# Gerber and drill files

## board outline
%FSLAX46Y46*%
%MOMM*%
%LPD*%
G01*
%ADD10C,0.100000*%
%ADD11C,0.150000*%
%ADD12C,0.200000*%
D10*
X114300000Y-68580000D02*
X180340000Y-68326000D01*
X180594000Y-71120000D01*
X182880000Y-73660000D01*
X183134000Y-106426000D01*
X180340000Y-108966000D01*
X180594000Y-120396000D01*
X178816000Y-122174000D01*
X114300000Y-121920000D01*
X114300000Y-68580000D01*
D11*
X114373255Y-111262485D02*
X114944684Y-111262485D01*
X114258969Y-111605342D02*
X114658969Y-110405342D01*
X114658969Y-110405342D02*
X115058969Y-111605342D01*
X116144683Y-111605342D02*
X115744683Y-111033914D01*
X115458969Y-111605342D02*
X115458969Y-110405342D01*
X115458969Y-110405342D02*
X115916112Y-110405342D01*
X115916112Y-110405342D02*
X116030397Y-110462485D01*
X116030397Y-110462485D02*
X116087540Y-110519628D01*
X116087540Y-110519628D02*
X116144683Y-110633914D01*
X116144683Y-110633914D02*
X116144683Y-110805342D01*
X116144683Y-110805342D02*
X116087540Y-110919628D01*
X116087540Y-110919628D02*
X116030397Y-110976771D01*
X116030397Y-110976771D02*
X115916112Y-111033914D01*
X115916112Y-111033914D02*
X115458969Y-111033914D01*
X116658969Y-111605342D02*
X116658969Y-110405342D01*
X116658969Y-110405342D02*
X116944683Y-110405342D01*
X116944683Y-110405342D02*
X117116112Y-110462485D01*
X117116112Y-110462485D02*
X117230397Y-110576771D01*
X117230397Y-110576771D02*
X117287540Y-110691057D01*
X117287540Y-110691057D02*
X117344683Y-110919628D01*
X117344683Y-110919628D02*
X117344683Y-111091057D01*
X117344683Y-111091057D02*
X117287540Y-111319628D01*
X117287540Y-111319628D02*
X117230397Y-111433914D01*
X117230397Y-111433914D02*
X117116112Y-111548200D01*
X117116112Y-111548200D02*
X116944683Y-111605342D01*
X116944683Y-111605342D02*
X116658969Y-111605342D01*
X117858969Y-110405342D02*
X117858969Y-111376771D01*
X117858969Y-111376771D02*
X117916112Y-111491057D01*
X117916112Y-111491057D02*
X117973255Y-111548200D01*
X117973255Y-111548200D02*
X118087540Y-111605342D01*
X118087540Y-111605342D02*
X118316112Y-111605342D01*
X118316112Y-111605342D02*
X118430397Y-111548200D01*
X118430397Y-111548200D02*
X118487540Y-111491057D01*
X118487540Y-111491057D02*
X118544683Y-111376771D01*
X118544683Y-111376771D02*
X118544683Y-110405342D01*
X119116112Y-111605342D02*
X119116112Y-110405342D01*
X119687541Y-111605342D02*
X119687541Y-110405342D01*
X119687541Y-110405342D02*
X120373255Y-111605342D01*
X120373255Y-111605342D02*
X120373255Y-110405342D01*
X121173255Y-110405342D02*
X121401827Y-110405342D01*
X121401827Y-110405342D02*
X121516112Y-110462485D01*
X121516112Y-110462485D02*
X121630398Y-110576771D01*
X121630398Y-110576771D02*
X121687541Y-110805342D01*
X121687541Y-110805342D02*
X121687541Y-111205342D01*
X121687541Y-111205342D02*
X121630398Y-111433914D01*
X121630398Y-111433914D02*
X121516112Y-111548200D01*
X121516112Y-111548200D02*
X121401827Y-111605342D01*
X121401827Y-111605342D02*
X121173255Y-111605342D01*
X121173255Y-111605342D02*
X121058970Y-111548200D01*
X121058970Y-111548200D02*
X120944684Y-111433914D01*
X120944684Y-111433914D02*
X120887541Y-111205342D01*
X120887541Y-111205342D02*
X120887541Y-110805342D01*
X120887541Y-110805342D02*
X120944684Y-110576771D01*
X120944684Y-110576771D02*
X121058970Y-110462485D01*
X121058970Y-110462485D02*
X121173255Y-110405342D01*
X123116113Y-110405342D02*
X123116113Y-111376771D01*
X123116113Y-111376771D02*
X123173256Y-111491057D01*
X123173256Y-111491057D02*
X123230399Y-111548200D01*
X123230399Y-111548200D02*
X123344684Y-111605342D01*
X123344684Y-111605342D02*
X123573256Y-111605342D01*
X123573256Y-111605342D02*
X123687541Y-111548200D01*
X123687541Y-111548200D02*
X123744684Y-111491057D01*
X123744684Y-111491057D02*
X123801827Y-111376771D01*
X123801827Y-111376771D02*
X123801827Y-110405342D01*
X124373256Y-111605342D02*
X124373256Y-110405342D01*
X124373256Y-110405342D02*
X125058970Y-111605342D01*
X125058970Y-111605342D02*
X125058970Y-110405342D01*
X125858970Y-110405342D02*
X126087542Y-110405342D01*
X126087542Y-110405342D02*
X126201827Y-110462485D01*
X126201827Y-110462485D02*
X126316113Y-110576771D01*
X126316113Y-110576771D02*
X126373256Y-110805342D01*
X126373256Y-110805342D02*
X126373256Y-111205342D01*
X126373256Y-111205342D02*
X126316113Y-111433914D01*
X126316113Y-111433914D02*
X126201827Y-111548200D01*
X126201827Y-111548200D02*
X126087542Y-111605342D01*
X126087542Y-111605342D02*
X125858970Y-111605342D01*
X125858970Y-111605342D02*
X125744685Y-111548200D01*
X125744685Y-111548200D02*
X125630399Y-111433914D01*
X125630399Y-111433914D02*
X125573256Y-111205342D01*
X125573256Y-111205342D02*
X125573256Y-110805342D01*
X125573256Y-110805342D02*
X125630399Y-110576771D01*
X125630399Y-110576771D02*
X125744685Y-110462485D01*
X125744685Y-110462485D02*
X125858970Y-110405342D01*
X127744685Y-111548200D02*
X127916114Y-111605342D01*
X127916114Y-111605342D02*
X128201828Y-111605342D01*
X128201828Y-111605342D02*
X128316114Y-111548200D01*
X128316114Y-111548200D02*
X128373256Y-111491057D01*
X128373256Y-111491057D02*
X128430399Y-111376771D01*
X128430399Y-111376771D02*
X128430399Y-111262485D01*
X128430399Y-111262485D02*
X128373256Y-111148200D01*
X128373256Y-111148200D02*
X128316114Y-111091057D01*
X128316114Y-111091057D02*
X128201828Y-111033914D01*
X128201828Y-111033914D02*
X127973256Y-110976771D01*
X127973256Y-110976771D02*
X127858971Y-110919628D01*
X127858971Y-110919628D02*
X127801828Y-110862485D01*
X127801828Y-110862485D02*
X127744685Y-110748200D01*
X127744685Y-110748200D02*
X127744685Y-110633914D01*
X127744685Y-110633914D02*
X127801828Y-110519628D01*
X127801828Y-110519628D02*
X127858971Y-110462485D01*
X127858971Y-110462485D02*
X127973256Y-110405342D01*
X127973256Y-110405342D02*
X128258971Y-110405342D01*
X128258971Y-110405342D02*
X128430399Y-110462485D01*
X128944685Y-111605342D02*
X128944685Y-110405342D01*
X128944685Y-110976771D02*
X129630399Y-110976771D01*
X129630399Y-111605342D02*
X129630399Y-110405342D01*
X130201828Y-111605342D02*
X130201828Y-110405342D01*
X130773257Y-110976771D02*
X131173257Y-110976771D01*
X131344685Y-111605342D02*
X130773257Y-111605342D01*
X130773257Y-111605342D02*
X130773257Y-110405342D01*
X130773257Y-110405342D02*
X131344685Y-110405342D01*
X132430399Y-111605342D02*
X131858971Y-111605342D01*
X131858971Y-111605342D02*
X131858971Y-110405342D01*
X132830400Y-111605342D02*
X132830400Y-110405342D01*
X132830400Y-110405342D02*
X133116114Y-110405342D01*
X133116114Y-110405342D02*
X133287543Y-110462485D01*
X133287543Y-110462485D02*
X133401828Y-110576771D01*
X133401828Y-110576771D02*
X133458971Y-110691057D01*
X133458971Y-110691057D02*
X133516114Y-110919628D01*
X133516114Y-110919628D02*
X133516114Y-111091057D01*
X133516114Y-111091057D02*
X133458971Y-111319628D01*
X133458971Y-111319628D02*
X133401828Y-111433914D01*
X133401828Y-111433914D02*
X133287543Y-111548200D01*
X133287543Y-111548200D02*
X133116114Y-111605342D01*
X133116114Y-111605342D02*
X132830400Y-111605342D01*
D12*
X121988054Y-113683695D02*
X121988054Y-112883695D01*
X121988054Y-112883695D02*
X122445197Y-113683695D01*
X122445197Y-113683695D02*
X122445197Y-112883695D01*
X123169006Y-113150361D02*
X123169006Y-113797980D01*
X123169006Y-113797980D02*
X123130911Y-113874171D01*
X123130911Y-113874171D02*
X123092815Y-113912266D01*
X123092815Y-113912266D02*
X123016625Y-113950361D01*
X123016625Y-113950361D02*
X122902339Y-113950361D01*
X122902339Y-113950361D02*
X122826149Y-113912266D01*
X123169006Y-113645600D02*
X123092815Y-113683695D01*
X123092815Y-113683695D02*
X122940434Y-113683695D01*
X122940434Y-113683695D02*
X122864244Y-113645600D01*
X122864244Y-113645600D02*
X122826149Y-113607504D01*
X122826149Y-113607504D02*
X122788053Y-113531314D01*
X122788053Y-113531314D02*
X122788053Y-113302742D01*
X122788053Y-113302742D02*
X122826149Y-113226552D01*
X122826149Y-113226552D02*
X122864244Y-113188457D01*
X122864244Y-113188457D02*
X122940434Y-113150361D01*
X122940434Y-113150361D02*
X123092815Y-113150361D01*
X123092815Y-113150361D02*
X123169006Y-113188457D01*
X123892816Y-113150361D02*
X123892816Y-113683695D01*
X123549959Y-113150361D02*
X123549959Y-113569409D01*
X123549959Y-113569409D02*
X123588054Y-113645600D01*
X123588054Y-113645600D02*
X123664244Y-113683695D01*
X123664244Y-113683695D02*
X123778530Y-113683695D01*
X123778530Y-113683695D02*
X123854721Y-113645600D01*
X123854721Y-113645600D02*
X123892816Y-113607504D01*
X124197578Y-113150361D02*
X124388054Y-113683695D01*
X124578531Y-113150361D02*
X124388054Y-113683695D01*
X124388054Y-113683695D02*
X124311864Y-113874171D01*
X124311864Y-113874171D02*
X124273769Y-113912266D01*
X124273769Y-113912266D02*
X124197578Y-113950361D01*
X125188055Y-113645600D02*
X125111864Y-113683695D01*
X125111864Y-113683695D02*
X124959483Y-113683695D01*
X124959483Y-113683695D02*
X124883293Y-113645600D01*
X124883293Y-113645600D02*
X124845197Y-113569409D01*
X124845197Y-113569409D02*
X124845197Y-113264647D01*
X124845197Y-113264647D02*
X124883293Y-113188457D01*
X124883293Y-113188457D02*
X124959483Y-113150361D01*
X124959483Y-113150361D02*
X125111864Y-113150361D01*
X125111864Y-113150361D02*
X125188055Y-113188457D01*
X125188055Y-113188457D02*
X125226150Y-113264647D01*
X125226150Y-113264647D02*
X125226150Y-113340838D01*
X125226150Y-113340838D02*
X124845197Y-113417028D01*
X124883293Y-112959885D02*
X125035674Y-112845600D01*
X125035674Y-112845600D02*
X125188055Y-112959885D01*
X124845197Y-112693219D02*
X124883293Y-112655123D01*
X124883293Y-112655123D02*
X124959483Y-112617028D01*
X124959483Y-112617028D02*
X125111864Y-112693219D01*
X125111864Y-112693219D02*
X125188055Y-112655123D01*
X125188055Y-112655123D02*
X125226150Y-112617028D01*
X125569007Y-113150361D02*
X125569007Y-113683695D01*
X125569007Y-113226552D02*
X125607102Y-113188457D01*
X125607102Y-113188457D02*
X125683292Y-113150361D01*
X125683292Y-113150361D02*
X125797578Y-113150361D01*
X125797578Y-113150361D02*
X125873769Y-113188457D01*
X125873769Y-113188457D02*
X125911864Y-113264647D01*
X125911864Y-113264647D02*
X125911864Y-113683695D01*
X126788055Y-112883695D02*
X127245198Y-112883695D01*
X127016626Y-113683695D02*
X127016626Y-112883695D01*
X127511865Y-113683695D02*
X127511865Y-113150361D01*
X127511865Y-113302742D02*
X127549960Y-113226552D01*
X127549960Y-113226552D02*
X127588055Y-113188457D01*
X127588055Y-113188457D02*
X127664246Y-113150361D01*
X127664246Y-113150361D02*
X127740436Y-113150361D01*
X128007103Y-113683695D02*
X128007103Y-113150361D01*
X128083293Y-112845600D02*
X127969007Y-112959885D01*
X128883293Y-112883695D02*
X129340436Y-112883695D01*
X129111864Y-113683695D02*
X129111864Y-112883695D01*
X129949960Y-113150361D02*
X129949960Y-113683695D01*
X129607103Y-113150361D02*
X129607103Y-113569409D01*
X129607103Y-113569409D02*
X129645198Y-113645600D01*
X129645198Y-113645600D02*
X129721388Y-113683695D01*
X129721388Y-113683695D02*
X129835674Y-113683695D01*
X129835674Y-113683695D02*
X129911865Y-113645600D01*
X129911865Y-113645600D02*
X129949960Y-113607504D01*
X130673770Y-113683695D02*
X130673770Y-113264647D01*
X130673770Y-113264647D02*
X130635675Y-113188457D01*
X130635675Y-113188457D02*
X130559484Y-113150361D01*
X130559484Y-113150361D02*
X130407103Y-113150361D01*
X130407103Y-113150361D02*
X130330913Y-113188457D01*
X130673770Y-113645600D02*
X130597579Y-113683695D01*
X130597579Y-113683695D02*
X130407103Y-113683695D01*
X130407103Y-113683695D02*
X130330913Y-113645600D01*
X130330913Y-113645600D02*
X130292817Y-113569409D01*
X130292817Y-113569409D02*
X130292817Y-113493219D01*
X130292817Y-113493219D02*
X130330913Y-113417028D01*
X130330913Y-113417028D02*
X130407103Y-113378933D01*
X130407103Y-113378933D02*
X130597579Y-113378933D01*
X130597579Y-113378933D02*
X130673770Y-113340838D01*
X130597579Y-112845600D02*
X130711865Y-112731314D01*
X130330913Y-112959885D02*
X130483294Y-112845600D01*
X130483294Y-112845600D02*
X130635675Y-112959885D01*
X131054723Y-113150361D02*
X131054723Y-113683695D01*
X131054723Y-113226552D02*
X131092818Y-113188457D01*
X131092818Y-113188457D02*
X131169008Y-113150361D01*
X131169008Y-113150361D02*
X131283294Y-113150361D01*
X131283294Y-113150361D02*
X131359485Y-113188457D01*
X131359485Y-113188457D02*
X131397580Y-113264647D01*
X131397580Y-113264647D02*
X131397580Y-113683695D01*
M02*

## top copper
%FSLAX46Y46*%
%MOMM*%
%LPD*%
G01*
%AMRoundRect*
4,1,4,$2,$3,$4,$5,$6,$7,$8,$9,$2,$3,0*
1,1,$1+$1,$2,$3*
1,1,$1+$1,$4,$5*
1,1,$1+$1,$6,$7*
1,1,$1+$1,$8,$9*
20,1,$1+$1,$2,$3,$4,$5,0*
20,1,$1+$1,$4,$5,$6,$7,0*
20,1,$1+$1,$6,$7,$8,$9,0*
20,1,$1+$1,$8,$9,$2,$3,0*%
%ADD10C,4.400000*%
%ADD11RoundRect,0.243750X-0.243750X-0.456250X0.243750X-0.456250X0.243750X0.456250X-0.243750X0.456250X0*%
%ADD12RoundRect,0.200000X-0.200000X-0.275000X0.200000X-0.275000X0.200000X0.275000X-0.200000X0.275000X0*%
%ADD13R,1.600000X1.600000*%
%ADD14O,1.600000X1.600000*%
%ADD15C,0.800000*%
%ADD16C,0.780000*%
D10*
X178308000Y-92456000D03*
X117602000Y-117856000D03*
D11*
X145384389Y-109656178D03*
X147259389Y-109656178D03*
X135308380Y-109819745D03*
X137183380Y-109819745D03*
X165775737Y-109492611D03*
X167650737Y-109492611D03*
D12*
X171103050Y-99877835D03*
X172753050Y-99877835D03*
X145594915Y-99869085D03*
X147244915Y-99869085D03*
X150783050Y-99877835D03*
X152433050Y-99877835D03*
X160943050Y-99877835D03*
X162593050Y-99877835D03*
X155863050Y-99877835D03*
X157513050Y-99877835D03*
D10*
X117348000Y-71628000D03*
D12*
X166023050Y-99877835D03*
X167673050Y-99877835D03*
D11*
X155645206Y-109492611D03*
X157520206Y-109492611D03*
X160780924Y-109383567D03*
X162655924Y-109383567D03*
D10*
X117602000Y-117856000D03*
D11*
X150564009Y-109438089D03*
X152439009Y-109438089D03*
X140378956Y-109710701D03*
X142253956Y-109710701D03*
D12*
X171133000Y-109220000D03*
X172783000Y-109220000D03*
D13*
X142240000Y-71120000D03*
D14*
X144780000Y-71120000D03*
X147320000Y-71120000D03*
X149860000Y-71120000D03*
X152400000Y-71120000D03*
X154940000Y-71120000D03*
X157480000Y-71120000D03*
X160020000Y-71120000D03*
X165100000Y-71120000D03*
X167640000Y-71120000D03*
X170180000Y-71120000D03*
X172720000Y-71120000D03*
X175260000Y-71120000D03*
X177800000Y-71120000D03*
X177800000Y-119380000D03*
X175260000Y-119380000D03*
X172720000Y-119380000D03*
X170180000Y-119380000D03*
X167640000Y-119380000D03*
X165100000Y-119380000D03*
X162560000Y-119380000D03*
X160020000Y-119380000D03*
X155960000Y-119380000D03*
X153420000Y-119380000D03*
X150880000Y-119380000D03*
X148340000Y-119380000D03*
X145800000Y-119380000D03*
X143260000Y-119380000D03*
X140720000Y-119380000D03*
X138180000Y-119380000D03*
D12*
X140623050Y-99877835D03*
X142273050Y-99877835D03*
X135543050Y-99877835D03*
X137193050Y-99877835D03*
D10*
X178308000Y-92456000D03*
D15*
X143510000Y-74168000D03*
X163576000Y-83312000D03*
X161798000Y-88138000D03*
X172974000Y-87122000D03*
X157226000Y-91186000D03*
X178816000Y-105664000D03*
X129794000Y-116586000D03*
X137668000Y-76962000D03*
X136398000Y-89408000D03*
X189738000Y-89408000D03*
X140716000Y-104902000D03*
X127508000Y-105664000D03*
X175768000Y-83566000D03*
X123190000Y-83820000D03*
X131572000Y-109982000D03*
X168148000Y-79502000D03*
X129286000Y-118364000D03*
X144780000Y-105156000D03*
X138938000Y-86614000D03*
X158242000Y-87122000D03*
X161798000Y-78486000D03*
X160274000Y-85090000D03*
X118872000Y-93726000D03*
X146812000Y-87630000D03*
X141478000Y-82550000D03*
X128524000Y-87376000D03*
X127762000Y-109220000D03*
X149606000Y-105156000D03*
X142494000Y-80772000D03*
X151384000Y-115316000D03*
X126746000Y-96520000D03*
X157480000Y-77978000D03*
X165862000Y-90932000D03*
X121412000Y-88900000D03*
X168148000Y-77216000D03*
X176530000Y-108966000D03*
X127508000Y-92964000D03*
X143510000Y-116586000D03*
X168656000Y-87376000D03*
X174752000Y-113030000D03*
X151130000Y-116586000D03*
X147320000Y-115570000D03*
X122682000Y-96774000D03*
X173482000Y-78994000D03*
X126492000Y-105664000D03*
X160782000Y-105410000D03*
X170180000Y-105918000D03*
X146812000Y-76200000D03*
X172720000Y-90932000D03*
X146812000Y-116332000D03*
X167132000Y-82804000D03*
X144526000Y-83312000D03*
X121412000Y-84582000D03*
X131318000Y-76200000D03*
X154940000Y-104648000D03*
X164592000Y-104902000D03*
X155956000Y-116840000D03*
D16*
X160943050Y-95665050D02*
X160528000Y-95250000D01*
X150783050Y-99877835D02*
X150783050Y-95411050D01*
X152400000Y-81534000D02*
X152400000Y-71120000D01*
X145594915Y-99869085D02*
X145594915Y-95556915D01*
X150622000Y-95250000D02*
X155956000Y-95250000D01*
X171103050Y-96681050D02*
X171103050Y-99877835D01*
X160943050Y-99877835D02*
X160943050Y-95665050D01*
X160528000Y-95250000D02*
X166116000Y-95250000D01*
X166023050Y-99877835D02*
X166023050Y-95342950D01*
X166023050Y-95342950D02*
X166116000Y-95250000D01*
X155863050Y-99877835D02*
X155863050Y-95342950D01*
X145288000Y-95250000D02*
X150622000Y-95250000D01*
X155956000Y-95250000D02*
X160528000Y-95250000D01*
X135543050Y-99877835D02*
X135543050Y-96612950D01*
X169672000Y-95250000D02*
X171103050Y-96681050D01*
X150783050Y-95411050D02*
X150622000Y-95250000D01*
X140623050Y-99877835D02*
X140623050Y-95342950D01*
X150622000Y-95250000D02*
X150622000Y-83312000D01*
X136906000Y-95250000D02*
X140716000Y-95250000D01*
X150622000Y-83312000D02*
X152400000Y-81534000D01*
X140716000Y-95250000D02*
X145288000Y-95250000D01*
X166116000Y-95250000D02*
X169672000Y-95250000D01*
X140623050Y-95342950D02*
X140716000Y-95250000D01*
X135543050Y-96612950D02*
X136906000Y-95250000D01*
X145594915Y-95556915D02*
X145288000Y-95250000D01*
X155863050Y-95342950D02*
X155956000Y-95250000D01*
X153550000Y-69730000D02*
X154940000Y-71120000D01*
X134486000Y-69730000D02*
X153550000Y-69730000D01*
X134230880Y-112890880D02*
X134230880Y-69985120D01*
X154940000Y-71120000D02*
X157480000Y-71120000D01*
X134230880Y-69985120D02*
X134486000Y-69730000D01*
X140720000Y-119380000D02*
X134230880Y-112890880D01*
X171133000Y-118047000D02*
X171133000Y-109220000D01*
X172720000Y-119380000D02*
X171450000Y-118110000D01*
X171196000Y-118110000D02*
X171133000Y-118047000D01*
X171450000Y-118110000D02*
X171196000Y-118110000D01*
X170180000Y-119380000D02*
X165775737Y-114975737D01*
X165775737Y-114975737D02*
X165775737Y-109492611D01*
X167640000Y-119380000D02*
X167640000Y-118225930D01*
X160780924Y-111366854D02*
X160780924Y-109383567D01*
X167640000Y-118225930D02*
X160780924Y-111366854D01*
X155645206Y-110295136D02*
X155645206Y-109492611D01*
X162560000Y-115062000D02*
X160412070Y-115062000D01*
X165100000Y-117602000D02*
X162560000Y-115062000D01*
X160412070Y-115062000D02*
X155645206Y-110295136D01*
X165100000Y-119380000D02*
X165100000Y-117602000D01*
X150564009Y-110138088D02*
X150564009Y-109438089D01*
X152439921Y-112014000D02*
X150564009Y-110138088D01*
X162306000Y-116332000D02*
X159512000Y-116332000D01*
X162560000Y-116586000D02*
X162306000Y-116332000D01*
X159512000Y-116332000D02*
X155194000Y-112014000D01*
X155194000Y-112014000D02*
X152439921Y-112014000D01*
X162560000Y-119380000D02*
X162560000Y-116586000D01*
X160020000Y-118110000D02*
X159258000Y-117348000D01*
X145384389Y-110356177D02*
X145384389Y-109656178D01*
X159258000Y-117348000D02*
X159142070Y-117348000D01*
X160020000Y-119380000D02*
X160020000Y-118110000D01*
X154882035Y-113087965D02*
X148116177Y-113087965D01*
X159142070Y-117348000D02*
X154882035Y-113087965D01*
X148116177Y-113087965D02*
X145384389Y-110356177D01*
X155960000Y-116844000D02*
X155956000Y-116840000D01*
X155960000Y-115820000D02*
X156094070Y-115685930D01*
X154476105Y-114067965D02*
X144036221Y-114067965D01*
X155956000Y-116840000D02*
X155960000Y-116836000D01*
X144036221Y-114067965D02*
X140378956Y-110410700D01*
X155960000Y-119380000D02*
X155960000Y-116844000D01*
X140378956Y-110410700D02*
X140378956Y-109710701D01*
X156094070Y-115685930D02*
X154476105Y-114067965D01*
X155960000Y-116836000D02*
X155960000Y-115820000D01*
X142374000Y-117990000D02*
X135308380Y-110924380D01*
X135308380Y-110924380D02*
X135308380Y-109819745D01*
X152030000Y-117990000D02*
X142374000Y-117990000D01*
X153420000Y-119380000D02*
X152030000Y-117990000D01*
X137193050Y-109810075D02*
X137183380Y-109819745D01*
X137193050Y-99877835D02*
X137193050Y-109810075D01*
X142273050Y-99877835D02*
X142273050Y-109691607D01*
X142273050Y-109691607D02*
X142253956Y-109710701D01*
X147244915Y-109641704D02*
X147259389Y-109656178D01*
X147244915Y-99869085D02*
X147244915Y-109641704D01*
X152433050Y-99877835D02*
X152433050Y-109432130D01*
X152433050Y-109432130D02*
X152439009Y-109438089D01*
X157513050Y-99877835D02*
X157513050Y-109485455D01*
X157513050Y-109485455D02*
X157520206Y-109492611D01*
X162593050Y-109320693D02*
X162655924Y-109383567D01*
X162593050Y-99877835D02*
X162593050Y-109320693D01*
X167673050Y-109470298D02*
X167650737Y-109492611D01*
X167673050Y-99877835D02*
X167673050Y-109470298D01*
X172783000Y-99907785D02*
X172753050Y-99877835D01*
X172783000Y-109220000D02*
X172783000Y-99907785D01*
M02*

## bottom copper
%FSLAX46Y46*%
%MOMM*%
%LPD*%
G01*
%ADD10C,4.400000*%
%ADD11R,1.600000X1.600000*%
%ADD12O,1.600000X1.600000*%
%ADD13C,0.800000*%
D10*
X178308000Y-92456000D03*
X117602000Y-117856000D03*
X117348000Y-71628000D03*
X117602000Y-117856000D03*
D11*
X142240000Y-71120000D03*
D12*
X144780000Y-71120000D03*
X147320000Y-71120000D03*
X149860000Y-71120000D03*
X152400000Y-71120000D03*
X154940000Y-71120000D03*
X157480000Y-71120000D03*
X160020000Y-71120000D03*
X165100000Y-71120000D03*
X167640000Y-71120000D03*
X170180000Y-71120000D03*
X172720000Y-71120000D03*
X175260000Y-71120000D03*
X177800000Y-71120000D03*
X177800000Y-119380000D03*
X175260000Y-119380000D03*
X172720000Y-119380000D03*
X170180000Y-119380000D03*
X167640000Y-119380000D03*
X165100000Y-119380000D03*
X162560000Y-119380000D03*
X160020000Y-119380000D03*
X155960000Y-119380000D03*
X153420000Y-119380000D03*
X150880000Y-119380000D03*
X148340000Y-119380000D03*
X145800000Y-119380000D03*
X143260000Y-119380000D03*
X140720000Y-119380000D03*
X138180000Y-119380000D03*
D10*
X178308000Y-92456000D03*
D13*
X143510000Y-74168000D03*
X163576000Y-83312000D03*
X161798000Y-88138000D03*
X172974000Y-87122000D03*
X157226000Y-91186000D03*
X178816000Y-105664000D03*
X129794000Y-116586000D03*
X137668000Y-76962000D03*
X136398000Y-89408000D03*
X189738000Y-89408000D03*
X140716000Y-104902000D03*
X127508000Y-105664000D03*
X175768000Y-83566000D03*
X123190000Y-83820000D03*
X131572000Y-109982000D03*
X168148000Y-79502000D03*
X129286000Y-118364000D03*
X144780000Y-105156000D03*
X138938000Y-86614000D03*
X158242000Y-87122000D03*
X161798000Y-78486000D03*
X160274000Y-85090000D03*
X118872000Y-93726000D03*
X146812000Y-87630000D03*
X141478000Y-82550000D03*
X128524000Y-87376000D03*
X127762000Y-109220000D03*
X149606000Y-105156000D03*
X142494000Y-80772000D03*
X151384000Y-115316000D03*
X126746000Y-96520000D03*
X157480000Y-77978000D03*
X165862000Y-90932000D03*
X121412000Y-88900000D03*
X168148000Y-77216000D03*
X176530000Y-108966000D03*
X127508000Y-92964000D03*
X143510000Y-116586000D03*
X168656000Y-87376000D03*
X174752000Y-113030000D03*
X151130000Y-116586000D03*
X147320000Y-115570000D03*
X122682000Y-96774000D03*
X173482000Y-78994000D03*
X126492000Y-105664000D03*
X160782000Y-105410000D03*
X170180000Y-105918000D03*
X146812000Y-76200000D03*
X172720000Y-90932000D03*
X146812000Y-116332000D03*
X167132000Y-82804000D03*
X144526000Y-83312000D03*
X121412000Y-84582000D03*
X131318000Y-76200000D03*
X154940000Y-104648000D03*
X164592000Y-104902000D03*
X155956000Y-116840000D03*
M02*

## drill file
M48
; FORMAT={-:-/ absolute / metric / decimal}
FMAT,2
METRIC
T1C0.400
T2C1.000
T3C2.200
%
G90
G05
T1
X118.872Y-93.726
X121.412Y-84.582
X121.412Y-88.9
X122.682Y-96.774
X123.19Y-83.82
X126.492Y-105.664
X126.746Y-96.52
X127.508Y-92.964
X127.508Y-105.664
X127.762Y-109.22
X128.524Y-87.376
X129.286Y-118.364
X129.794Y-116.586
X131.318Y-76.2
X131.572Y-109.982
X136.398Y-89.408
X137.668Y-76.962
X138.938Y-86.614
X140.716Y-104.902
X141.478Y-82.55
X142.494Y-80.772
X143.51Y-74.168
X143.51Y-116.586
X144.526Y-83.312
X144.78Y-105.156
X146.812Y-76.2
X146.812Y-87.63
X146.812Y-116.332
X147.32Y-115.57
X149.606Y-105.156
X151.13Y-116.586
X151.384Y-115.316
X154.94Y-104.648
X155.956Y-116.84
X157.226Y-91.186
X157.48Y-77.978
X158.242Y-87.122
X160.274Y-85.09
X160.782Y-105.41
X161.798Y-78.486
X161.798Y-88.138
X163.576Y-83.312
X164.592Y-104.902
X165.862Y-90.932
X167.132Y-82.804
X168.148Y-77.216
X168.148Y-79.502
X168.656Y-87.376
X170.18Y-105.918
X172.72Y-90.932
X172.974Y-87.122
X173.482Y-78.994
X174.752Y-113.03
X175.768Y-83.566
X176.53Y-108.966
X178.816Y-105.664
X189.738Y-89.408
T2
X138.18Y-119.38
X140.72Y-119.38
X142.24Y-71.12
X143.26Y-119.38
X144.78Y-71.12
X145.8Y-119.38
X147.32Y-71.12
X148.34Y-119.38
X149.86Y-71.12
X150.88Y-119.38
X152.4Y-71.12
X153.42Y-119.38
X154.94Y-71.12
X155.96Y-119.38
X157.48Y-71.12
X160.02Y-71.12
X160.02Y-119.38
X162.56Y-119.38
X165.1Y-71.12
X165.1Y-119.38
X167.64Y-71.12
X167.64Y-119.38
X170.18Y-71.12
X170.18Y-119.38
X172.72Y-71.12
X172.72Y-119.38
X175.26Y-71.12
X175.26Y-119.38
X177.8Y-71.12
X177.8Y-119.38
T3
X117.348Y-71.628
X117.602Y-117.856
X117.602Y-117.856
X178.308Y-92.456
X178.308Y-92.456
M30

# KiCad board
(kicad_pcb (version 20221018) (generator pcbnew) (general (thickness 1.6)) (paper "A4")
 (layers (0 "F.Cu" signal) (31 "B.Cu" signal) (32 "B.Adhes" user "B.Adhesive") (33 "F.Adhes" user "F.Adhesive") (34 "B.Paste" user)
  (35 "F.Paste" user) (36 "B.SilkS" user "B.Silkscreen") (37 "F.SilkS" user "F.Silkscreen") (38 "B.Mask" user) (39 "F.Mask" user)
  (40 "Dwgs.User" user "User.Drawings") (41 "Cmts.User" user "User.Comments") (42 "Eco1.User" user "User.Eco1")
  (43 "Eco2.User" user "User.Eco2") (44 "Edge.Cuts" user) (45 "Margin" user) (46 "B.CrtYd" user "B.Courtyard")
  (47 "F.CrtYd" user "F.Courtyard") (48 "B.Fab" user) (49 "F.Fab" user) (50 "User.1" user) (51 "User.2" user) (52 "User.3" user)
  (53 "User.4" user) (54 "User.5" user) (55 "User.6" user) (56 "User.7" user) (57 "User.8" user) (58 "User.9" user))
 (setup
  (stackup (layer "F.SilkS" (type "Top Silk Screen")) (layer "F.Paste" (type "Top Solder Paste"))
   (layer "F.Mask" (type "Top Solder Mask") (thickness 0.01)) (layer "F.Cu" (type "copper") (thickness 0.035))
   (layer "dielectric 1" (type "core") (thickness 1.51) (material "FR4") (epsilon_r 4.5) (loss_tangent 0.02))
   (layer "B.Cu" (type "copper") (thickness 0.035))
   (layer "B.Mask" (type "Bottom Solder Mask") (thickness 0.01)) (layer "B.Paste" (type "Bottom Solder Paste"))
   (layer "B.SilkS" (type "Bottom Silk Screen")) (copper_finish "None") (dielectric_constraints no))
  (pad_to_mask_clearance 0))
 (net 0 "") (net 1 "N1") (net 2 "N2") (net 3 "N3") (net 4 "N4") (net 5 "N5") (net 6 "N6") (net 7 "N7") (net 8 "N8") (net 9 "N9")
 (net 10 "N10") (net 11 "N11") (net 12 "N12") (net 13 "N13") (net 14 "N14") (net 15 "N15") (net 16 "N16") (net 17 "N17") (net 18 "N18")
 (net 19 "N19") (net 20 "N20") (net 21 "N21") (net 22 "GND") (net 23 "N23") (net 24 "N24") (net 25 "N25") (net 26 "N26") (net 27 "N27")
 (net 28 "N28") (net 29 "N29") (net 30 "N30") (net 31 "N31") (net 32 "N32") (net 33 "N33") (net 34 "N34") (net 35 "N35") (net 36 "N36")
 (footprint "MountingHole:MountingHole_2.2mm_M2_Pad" (layer "F.Cu") (at 178.308 92.456)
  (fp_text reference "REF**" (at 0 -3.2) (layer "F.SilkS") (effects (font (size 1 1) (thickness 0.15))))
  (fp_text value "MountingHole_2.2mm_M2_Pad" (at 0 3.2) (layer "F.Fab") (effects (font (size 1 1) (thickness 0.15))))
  (pad "1" thru_hole circle (at 0 0) (size 4.4 4.4) (drill 2.2) (layers "*.Cu" "*.Mask")))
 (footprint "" (layer "F.Cu") (at 117.602 117.856)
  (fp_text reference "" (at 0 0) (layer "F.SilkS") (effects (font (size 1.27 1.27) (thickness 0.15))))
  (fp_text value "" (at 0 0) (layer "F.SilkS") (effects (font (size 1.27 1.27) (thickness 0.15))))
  (pad "1" thru_hole circle (at 0 0) (size 4.4 4.4) (drill 2.2) (layers "*.Cu" "*.Mask")))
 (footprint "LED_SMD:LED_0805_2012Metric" (layer "F.Cu") (at 146.321889 109.656178)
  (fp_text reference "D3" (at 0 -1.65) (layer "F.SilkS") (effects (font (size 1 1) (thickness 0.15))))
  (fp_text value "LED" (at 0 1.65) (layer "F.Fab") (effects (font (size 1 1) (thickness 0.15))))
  (pad "1" smd roundrect (at -0.9375 0) (size 0.975 1.4) (layers "F.Cu" "F.Paste" "F.Mask") (roundrect_rratio 0.25) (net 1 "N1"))
  (pad "2" smd roundrect (at 0.9375 0) (size 0.975 1.4) (layers "F.Cu" "F.Paste" "F.Mask") (roundrect_rratio 0.25) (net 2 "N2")))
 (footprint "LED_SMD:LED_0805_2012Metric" (layer "F.Cu") (at 136.24588 109.819745)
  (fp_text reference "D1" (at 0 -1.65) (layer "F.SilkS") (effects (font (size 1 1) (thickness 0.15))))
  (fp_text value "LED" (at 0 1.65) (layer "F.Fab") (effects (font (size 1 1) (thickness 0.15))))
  (pad "1" smd roundrect (at -0.9375 0) (size 0.975 1.4) (layers "F.Cu" "F.Paste" "F.Mask") (roundrect_rratio 0.25) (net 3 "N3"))
  (pad "2" smd roundrect (at 0.9375 0) (size 0.975 1.4) (layers "F.Cu" "F.Paste" "F.Mask") (roundrect_rratio 0.25) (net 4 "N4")))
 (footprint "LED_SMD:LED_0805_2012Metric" (layer "F.Cu") (at 166.713237 109.492611)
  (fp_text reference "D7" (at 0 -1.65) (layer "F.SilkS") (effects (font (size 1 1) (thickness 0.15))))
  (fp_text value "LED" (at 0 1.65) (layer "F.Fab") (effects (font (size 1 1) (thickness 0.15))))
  (pad "1" smd roundrect (at -0.9375 0) (size 0.975 1.4) (layers "F.Cu" "F.Paste" "F.Mask") (roundrect_rratio 0.25) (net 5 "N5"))
  (pad "2" smd roundrect (at 0.9375 0) (size 0.975 1.4) (layers "F.Cu" "F.Paste" "F.Mask") (roundrect_rratio 0.25) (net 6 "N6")))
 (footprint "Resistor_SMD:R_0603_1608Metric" (layer "F.Cu") (at 171.92805 99.877835)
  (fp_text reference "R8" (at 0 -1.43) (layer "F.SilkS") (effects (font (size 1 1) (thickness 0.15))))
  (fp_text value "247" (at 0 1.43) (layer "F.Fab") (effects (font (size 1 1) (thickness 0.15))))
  (pad "1" smd roundrect (at -0.825 0) (size 0.8 0.95) (layers "F.Cu" "F.Paste" "F.Mask") (roundrect_rratio 0.25) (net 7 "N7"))
  (pad "2" smd roundrect (at 0.825 0) (size 0.8 0.95) (layers "F.Cu" "F.Paste" "F.Mask") (roundrect_rratio 0.25) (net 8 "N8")))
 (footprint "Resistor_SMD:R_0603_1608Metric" (layer "F.Cu") (at 146.419915 99.869085)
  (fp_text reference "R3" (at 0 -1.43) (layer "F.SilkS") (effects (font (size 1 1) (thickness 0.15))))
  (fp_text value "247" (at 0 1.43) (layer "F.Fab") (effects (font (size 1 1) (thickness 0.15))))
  (pad "1" smd roundrect (at -0.825 0) (size 0.8 0.95) (layers "F.Cu" "F.Paste" "F.Mask") (roundrect_rratio 0.25) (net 7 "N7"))
  (pad "2" smd roundrect (at 0.825 0) (size 0.8 0.95) (layers "F.Cu" "F.Paste" "F.Mask") (roundrect_rratio 0.25) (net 2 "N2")))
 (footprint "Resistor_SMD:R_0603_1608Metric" (layer "F.Cu") (at 151.60805 99.877835)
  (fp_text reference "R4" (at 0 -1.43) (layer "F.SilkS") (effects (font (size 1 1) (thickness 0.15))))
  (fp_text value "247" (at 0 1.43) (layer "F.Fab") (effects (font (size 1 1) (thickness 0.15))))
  (pad "1" smd roundrect (at -0.825 0) (size 0.8 0.95) (layers "F.Cu" "F.Paste" "F.Mask") (roundrect_rratio 0.25) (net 7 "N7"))
  (pad "2" smd roundrect (at 0.825 0) (size 0.8 0.95) (layers "F.Cu" "F.Paste" "F.Mask") (roundrect_rratio 0.25) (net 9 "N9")))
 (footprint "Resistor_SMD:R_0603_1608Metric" (layer "F.Cu") (at 161.76805 99.877835)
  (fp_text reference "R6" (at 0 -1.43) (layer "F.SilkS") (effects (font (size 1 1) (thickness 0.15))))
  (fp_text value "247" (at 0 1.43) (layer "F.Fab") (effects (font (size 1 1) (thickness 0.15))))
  (pad "1" smd roundrect (at -0.825 0) (size 0.8 0.95) (layers "F.Cu" "F.Paste" "F.Mask") (roundrect_rratio 0.25) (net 7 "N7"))
  (pad "2" smd roundrect (at 0.825 0) (size 0.8 0.95) (layers "F.Cu" "F.Paste" "F.Mask") (roundrect_rratio 0.25) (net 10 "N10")))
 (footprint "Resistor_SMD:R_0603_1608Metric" (layer "F.Cu") (at 156.68805 99.877835)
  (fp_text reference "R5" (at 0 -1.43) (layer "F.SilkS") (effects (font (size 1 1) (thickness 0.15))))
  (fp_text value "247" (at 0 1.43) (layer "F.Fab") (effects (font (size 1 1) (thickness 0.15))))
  (pad "1" smd roundrect (at -0.825 0) (size 0.8 0.95) (layers "F.Cu" "F.Paste" "F.Mask") (roundrect_rratio 0.25) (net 7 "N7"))
  (pad "2" smd roundrect (at 0.825 0) (size 0.8 0.95) (layers "F.Cu" "F.Paste" "F.Mask") (roundrect_rratio 0.25) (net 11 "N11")))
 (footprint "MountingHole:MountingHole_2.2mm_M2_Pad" (layer "F.Cu") (at 117.348 71.628)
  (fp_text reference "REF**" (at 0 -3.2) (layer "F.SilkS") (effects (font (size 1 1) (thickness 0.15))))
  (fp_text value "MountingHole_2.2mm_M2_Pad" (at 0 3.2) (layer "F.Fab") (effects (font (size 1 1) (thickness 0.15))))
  (pad "1" thru_hole circle (at 0 0) (size 4.4 4.4) (drill 2.2) (layers "*.Cu" "*.Mask")))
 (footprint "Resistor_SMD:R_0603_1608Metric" (layer "F.Cu") (at 166.84805 99.877835)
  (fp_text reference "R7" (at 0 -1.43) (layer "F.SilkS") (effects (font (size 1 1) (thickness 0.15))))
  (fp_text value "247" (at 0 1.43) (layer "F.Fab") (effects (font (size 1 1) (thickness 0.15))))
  (pad "1" smd roundrect (at -0.825 0) (size 0.8 0.95) (layers "F.Cu" "F.Paste" "F.Mask") (roundrect_rratio 0.25) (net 7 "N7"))
  (pad "2" smd roundrect (at 0.825 0) (size 0.8 0.95) (layers "F.Cu" "F.Paste" "F.Mask") (roundrect_rratio 0.25) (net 6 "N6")))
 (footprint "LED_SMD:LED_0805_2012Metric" (layer "F.Cu") (at 156.582706 109.492611)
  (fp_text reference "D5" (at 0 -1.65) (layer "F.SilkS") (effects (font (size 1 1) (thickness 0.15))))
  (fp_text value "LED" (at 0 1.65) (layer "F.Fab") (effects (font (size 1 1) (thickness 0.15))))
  (pad "1" smd roundrect (at -0.9375 0) (size 0.975 1.4) (layers "F.Cu" "F.Paste" "F.Mask") (roundrect_rratio 0.25) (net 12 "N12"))
  (pad "2" smd roundrect (at 0.9375 0) (size 0.975 1.4) (layers "F.Cu" "F.Paste" "F.Mask") (roundrect_rratio 0.25) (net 11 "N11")))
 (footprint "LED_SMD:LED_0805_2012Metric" (layer "F.Cu") (at 161.718424 109.383567)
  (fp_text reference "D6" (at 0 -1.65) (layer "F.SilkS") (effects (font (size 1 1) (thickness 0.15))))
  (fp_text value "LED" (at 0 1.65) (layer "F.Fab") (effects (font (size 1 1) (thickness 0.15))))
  (pad "1" smd roundrect (at -0.9375 0) (size 0.975 1.4) (layers "F.Cu" "F.Paste" "F.Mask") (roundrect_rratio 0.25) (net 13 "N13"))
  (pad "2" smd roundrect (at 0.9375 0) (size 0.975 1.4) (layers "F.Cu" "F.Paste" "F.Mask") (roundrect_rratio 0.25) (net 10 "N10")))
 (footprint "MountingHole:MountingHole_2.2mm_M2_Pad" (layer "F.Cu") (at 117.602 117.856)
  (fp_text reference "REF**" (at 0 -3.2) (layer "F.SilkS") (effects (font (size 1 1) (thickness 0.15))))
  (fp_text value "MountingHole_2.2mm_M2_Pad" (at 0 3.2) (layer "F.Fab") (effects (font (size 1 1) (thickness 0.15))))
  (pad "1" thru_hole circle (at 0 0) (size 4.4 4.4) (drill 2.2) (layers "*.Cu" "*.Mask")))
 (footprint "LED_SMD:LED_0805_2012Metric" (layer "F.Cu") (at 151.501509 109.438089)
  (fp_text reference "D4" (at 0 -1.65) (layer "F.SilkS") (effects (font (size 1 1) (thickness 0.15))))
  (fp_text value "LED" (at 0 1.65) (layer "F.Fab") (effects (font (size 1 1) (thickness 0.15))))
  (pad "1" smd roundrect (at -0.9375 0) (size 0.975 1.4) (layers "F.Cu" "F.Paste" "F.Mask") (roundrect_rratio 0.25) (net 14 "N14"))
  (pad "2" smd roundrect (at 0.9375 0) (size 0.975 1.4) (layers "F.Cu" "F.Paste" "F.Mask") (roundrect_rratio 0.25) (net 9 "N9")))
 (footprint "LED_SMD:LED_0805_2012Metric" (layer "F.Cu") (at 141.316456 109.710701)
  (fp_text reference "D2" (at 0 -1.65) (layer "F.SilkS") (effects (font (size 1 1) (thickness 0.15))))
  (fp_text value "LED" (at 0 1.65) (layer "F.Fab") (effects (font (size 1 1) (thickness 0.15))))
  (pad "1" smd roundrect (at -0.9375 0) (size 0.975 1.4) (layers "F.Cu" "F.Paste" "F.Mask") (roundrect_rratio 0.25) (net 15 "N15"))
  (pad "2" smd roundrect (at 0.9375 0) (size 0.975 1.4) (layers "F.Cu" "F.Paste" "F.Mask") (roundrect_rratio 0.25) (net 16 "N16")))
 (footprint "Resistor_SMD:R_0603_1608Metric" (layer "F.Cu") (at 171.958 109.22)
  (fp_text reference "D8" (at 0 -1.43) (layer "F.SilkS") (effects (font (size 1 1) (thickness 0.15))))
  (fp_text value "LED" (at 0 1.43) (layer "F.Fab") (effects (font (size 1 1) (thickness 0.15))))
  (pad "1" smd roundrect (at -0.825 0) (size 0.8 0.95) (layers "F.Cu" "F.Paste" "F.Mask") (roundrect_rratio 0.25) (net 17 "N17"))
  (pad "2" smd roundrect (at 0.825 0) (size 0.8 0.95) (layers "F.Cu" "F.Paste" "F.Mask") (roundrect_rratio 0.25) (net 8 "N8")))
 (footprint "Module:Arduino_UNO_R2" (layer "F.Cu") (at 142.24 71.12)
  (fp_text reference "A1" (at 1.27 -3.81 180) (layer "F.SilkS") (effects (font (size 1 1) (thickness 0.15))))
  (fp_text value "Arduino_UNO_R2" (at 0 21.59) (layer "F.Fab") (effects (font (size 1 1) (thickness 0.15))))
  (pad "1" thru_hole rect (at 0 0 90) (size 1.6 1.6) (drill 1) (layers "*.Cu" "*.Mask") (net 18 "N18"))
  (pad "2" thru_hole oval (at 2.54 0 90) (size 1.6 1.6) (drill 1) (layers "*.Cu" "*.Mask") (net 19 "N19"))
  (pad "3" thru_hole oval (at 5.08 0 90) (size 1.6 1.6) (drill 1) (layers "*.Cu" "*.Mask") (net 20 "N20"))
  (pad "4" thru_hole oval (at 7.62 0 90) (size 1.6 1.6) (drill 1) (layers "*.Cu" "*.Mask") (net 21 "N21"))
  (pad "5" thru_hole oval (at 10.16 0 90) (size 1.6 1.6) (drill 1) (layers "*.Cu" "*.Mask") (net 7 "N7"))
  (pad "6" thru_hole oval (at 12.7 0 90) (size 1.6 1.6) (drill 1) (layers "*.Cu" "*.Mask") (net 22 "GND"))
  (pad "7" thru_hole oval (at 15.24 0 90) (size 1.6 1.6) (drill 1) (layers "*.Cu" "*.Mask") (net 22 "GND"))
  (pad "8" thru_hole oval (at 17.78 0 90) (size 1.6 1.6) (drill 1) (layers "*.Cu" "*.Mask") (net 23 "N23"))
  (pad "9" thru_hole oval (at 22.86 0 90) (size 1.6 1.6) (drill 1) (layers "*.Cu" "*.Mask") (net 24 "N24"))
  (pad "10" thru_hole oval (at 25.4 0 90) (size 1.6 1.6) (drill 1) (layers "*.Cu" "*.Mask") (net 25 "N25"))
  (pad "11" thru_hole oval (at 27.94 0 90) (size 1.6 1.6) (drill 1) (layers "*.Cu" "*.Mask") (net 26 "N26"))
  (pad "12" thru_hole oval (at 30.48 0 90) (size 1.6 1.6) (drill 1) (layers "*.Cu" "*.Mask") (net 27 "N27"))
  (pad "13" thru_hole oval (at 33.02 0 90) (size 1.6 1.6) (drill 1) (layers "*.Cu" "*.Mask") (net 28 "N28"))
  (pad "14" thru_hole oval (at 35.56 0 90) (size 1.6 1.6) (drill 1) (layers "*.Cu" "*.Mask") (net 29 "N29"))
  (pad "15" thru_hole oval (at 35.56 48.26 90) (size 1.6 1.6) (drill 1) (layers "*.Cu" "*.Mask") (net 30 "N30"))
  (pad "16" thru_hole oval (at 33.02 48.26 90) (size 1.6 1.6) (drill 1) (layers "*.Cu" "*.Mask") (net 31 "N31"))
  (pad "17" thru_hole oval (at 30.48 48.26 90) (size 1.6 1.6) (drill 1) (layers "*.Cu" "*.Mask") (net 17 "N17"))
  (pad "18" thru_hole oval (at 27.94 48.26 90) (size 1.6 1.6) (drill 1) (layers "*.Cu" "*.Mask") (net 5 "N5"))
  (pad "19" thru_hole oval (at 25.4 48.26 90) (size 1.6 1.6) (drill 1) (layers "*.Cu" "*.Mask") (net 13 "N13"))
  (pad "20" thru_hole oval (at 22.86 48.26 90) (size 1.6 1.6) (drill 1) (layers "*.Cu" "*.Mask") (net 12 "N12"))
  (pad "21" thru_hole oval (at 20.32 48.26 90) (size 1.6 1.6) (drill 1) (layers "*.Cu" "*.Mask") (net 14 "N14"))
  (pad "22" thru_hole oval (at 17.78 48.26 90) (size 1.6 1.6) (drill 1) (layers "*.Cu" "*.Mask") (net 1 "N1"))
  (pad "23" thru_hole oval (at 13.72 48.26 90) (size 1.6 1.6) (drill 1) (layers "*.Cu" "*.Mask") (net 15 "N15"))
  (pad "24" thru_hole oval (at 11.18 48.26 90) (size 1.6 1.6) (drill 1) (layers "*.Cu" "*.Mask") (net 3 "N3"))
  (pad "25" thru_hole oval (at 8.64 48.26 90) (size 1.6 1.6) (drill 1) (layers "*.Cu" "*.Mask") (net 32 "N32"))
  (pad "26" thru_hole oval (at 6.1 48.26 90) (size 1.6 1.6) (drill 1) (layers "*.Cu" "*.Mask") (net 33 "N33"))
  (pad "27" thru_hole oval (at 3.56 48.26 90) (size 1.6 1.6) (drill 1) (layers "*.Cu" "*.Mask") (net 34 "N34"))
  (pad "28" thru_hole oval (at 1.02 48.26 90) (size 1.6 1.6) (drill 1) (layers "*.Cu" "*.Mask") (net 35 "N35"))
  (pad "29" thru_hole oval (at -1.52 48.26 90) (size 1.6 1.6) (drill 1) (layers "*.Cu" "*.Mask") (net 22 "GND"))
  (pad "30" thru_hole oval (at -4.06 48.26 90) (size 1.6 1.6) (drill 1) (layers "*.Cu" "*.Mask") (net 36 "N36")))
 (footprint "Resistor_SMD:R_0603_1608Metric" (layer "F.Cu") (at 141.44805 99.877835)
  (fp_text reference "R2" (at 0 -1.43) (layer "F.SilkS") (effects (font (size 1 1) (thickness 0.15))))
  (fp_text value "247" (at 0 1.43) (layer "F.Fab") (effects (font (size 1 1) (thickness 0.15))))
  (pad "1" smd roundrect (at -0.825 0) (size 0.8 0.95) (layers "F.Cu" "F.Paste" "F.Mask") (roundrect_rratio 0.25) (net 7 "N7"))
  (pad "2" smd roundrect (at 0.825 0) (size 0.8 0.95) (layers "F.Cu" "F.Paste" "F.Mask") (roundrect_rratio 0.25) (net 16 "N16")))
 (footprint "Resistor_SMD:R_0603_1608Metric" (layer "F.Cu") (at 136.36805 99.877835)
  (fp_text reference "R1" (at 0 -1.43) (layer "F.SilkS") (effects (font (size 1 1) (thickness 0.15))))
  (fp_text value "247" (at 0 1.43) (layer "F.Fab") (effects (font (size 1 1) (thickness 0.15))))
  (pad "1" smd roundrect (at -0.825 0) (size 0.8 0.95) (layers "F.Cu" "F.Paste" "F.Mask") (roundrect_rratio 0.25) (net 7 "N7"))
  (pad "2" smd roundrect (at 0.825 0) (size 0.8 0.95) (layers "F.Cu" "F.Paste" "F.Mask") (roundrect_rratio 0.25) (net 4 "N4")))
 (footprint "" (layer "F.Cu") (at 178.308 92.456)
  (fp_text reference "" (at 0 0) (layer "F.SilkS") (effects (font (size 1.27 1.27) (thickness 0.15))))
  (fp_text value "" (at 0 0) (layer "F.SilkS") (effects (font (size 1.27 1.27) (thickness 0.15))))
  (pad "1" thru_hole circle (at 0 0) (size 4.4 4.4) (drill 2.2) (layers "*.Cu" "*.Mask")))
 (gr_poly
  (pts (xy 114.3 68.58) (xy 180.34 68.326) (xy 180.594 71.12) (xy 182.88 73.66) (xy 183.134 106.426) (xy 180.34 108.966)
   (xy 180.594 120.396) (xy 178.816 122.174) (xy 114.3 121.92))
  (stroke (width 0.1) (type solid)) (fill none) (layer "Edge.Cuts"))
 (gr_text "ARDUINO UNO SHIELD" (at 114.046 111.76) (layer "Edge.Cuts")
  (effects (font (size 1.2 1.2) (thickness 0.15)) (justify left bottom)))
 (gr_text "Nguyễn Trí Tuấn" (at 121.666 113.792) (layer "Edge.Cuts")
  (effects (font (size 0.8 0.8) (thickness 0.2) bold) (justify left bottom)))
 (via (at 143.51 74.168) (size 0.8) (drill 0.4) (layers "F.Cu" "B.Cu") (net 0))
 (via (at 163.576 83.312) (size 0.8) (drill 0.4) (layers "F.Cu" "B.Cu") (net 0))
 (via (at 161.798 88.138) (size 0.8) (drill 0.4) (layers "F.Cu" "B.Cu") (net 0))
 (via (at 172.974 87.122) (size 0.8) (drill 0.4) (layers "F.Cu" "B.Cu") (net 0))
 (via (at 157.226 91.186) (size 0.8) (drill 0.4) (layers "F.Cu" "B.Cu") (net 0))
 (via (at 178.816 105.664) (size 0.8) (drill 0.4) (layers "F.Cu" "B.Cu") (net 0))
 (via (at 129.794 116.586) (size 0.8) (drill 0.4) (layers "F.Cu" "B.Cu") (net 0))
 (via (at 137.668 76.962) (size 0.8) (drill 0.4) (layers "F.Cu" "B.Cu") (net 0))
 (via (at 136.398 89.408) (size 0.8) (drill 0.4) (layers "F.Cu" "B.Cu") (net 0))
 (via (at 189.738 89.408) (size 0.8) (drill 0.4) (layers "F.Cu" "B.Cu") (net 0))
 (via (at 140.716 104.902) (size 0.8) (drill 0.4) (layers "F.Cu" "B.Cu") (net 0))
 (via (at 127.508 105.664) (size 0.8) (drill 0.4) (layers "F.Cu" "B.Cu") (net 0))
 (via (at 175.768 83.566) (size 0.8) (drill 0.4) (layers "F.Cu" "B.Cu") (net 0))
 (via (at 123.19 83.82) (size 0.8) (drill 0.4) (layers "F.Cu" "B.Cu") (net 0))
 (via (at 131.572 109.982) (size 0.8) (drill 0.4) (layers "F.Cu" "B.Cu") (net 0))
 (via (at 168.148 79.502) (size 0.8) (drill 0.4) (layers "F.Cu" "B.Cu") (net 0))
 (via (at 129.286 118.364) (size 0.8) (drill 0.4) (layers "F.Cu" "B.Cu") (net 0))
 (via (at 144.78 105.156) (size 0.8) (drill 0.4) (layers "F.Cu" "B.Cu") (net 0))
 (via (at 138.938 86.614) (size 0.8) (drill 0.4) (layers "F.Cu" "B.Cu") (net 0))
 (via (at 158.242 87.122) (size 0.8) (drill 0.4) (layers "F.Cu" "B.Cu") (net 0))
 (via (at 161.798 78.486) (size 0.8) (drill 0.4) (layers "F.Cu" "B.Cu") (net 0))
 (via (at 160.274 85.09) (size 0.8) (drill 0.4) (layers "F.Cu" "B.Cu") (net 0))
 (via (at 118.872 93.726) (size 0.8) (drill 0.4) (layers "F.Cu" "B.Cu") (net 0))
 (via (at 146.812 87.63) (size 0.8) (drill 0.4) (layers "F.Cu" "B.Cu") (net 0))
 (via (at 141.478 82.55) (size 0.8) (drill 0.4) (layers "F.Cu" "B.Cu") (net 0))
 (via (at 128.524 87.376) (size 0.8) (drill 0.4) (layers "F.Cu" "B.Cu") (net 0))
 (via (at 127.762 109.22) (size 0.8) (drill 0.4) (layers "F.Cu" "B.Cu") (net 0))
 (via (at 149.606 105.156) (size 0.8) (drill 0.4) (layers "F.Cu" "B.Cu") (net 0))
 (via (at 142.494 80.772) (size 0.8) (drill 0.4) (layers "F.Cu" "B.Cu") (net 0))
 (via (at 151.384 115.316) (size 0.8) (drill 0.4) (layers "F.Cu" "B.Cu") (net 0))
 (via (at 126.746 96.52) (size 0.8) (drill 0.4) (layers "F.Cu" "B.Cu") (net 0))
 (via (at 157.48 77.978) (size 0.8) (drill 0.4) (layers "F.Cu" "B.Cu") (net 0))
 (via (at 165.862 90.932) (size 0.8) (drill 0.4) (layers "F.Cu" "B.Cu") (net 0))
 (via (at 121.412 88.9) (size 0.8) (drill 0.4) (layers "F.Cu" "B.Cu") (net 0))
 (via (at 168.148 77.216) (size 0.8) (drill 0.4) (layers "F.Cu" "B.Cu") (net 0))
 (via (at 176.53 108.966) (size 0.8) (drill 0.4) (layers "F.Cu" "B.Cu") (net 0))
 (via (at 127.508 92.964) (size 0.8) (drill 0.4) (layers "F.Cu" "B.Cu") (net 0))
 (via (at 143.51 116.586) (size 0.8) (drill 0.4) (layers "F.Cu" "B.Cu") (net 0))
 (via (at 168.656 87.376) (size 0.8) (drill 0.4) (layers "F.Cu" "B.Cu") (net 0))
 (via (at 174.752 113.03) (size 0.8) (drill 0.4) (layers "F.Cu" "B.Cu") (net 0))
 (via (at 151.13 116.586) (size 0.8) (drill 0.4) (layers "F.Cu" "B.Cu") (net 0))
 (via (at 147.32 115.57) (size 0.8) (drill 0.4) (layers "F.Cu" "B.Cu") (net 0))
 (via (at 122.682 96.774) (size 0.8) (drill 0.4) (layers "F.Cu" "B.Cu") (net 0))
 (via (at 173.482 78.994) (size 0.8) (drill 0.4) (layers "F.Cu" "B.Cu") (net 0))
 (via (at 126.492 105.664) (size 0.8) (drill 0.4) (layers "F.Cu" "B.Cu") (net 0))
 (via (at 160.782 105.41) (size 0.8) (drill 0.4) (layers "F.Cu" "B.Cu") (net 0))
 (via (at 170.18 105.918) (size 0.8) (drill 0.4) (layers "F.Cu" "B.Cu") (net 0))
 (via (at 146.812 76.2) (size 0.8) (drill 0.4) (layers "F.Cu" "B.Cu") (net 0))
 (via (at 172.72 90.932) (size 0.8) (drill 0.4) (layers "F.Cu" "B.Cu") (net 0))
 (via (at 146.812 116.332) (size 0.8) (drill 0.4) (layers "F.Cu" "B.Cu") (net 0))
 (via (at 167.132 82.804) (size 0.8) (drill 0.4) (layers "F.Cu" "B.Cu") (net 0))
 (via (at 144.526 83.312) (size 0.8) (drill 0.4) (layers "F.Cu" "B.Cu") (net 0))
 (via (at 121.412 84.582) (size 0.8) (drill 0.4) (layers "F.Cu" "B.Cu") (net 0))
 (via (at 131.318 76.2) (size 0.8) (drill 0.4) (layers "F.Cu" "B.Cu") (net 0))
 (via (at 154.94 104.648) (size 0.8) (drill 0.4) (layers "F.Cu" "B.Cu") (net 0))
 (via (at 164.592 104.902) (size 0.8) (drill 0.4) (layers "F.Cu" "B.Cu") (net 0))
 (segment (start 160.94305 95.66505) (end 160.528 95.25) (width 0.78) (layer "F.Cu") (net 7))
 (segment (start 150.78305 99.877835) (end 150.78305 95.41105) (width 0.78) (layer "F.Cu") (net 7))
 (segment (start 152.4 81.534) (end 152.4 71.12) (width 0.78) (layer "F.Cu") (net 7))
 (segment (start 145.594915 99.869085) (end 145.594915 95.556915) (width 0.78) (layer "F.Cu") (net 7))
 (segment (start 150.622 95.25) (end 155.956 95.25) (width 0.78) (layer "F.Cu") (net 7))
 (segment (start 171.10305 96.68105) (end 171.10305 99.877835) (width 0.78) (layer "F.Cu") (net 7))
 (segment (start 160.94305 99.877835) (end 160.94305 95.66505) (width 0.78) (layer "F.Cu") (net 7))
 (segment (start 160.528 95.25) (end 166.116 95.25) (width 0.78) (layer "F.Cu") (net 7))
 (segment (start 166.02305 99.877835) (end 166.02305 95.34295) (width 0.78) (layer "F.Cu") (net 7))
 (segment (start 166.02305 95.34295) (end 166.116 95.25) (width 0.78) (layer "F.Cu") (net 7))
 (segment (start 155.86305 99.877835) (end 155.86305 95.34295) (width 0.78) (layer "F.Cu") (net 7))
 (segment (start 145.288 95.25) (end 150.622 95.25) (width 0.78) (layer "F.Cu") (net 7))
 (segment (start 155.956 95.25) (end 160.528 95.25) (width 0.78) (layer "F.Cu") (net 7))
 (segment (start 135.54305 99.877835) (end 135.54305 96.61295) (width 0.78) (layer "F.Cu") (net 7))
 (segment (start 169.672 95.25) (end 171.10305 96.68105) (width 0.78) (layer "F.Cu") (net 7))
 (segment (start 150.78305 95.41105) (end 150.622 95.25) (width 0.78) (layer "F.Cu") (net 7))
 (segment (start 140.62305 99.877835) (end 140.62305 95.34295) (width 0.78) (layer "F.Cu") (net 7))
 (segment (start 150.622 95.25) (end 150.622 83.312) (width 0.78) (layer "F.Cu") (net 7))
 (segment (start 136.906 95.25) (end 140.716 95.25) (width 0.78) (layer "F.Cu") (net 7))
 (segment (start 150.622 83.312) (end 152.4 81.534) (width 0.78) (layer "F.Cu") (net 7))
 (segment (start 140.716 95.25) (end 145.288 95.25) (width 0.78) (layer "F.Cu") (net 7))
 (segment (start 166.116 95.25) (end 169.672 95.25) (width 0.78) (layer "F.Cu") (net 7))
 (segment (start 140.62305 95.34295) (end 140.716 95.25) (width 0.78) (layer "F.Cu") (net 7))
 (segment (start 135.54305 96.61295) (end 136.906 95.25) (width 0.78) (layer "F.Cu") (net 7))
 (segment (start 145.594915 95.556915) (end 145.288 95.25) (width 0.78) (layer "F.Cu") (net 7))
 (segment (start 155.86305 95.34295) (end 155.956 95.25) (width 0.78) (layer "F.Cu") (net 7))
 (segment (start 153.55 69.73) (end 154.94 71.12) (width 0.78) (layer "F.Cu") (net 22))
 (segment (start 134.486 69.73) (end 153.55 69.73) (width 0.78) (layer "F.Cu") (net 22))
 (segment (start 134.23088 112.89088) (end 134.23088 69.98512) (width 0.78) (layer "F.Cu") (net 22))
 (segment (start 154.94 71.12) (end 157.48 71.12) (width 0.78) (layer "F.Cu") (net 22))
 (segment (start 134.23088 69.98512) (end 134.486 69.73) (width 0.78) (layer "F.Cu") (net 22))
 (segment (start 140.72 119.38) (end 134.23088 112.89088) (width 0.78) (layer "F.Cu") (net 22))
 (segment (start 171.133 118.047) (end 171.133 109.22) (width 0.78) (layer "F.Cu") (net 17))
 (segment (start 172.72 119.38) (end 171.45 118.11) (width 0.78) (layer "F.Cu") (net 17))
 (segment (start 171.196 118.11) (end 171.133 118.047) (width 0.78) (layer "F.Cu") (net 17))
 (segment (start 171.45 118.11) (end 171.196 118.11) (width 0.78) (layer "F.Cu") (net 17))
 (segment (start 170.18 119.38) (end 165.775737 114.975737) (width 0.78) (layer "F.Cu") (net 5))
 (segment (start 165.775737 114.975737) (end 165.775737 109.492611) (width 0.78) (layer "F.Cu") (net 5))
 (segment (start 167.64 119.38) (end 167.64 118.22593) (width 0.78) (layer "F.Cu") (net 13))
 (segment (start 160.780924 111.366854) (end 160.780924 109.383567) (width 0.78) (layer "F.Cu") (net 13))
 (segment (start 167.64 118.22593) (end 160.780924 111.366854) (width 0.78) (layer "F.Cu") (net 13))
 (segment (start 155.645206 110.295136) (end 155.645206 109.492611) (width 0.78) (layer "F.Cu") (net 12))
 (segment (start 162.56 115.062) (end 160.41207 115.062) (width 0.78) (layer "F.Cu") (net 12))
 (segment (start 165.1 117.602) (end 162.56 115.062) (width 0.78) (layer "F.Cu") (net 12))
 (segment (start 160.41207 115.062) (end 155.645206 110.295136) (width 0.78) (layer "F.Cu") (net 12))
 (segment (start 165.1 119.38) (end 165.1 117.602) (width 0.78) (layer "F.Cu") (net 12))
 (segment (start 150.564009 110.138088) (end 150.564009 109.438089) (width 0.78) (layer "F.Cu") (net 14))
 (segment (start 152.439921 112.014) (end 150.564009 110.138088) (width 0.78) (layer "F.Cu") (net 14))
 (segment (start 162.306 116.332) (end 159.512 116.332) (width 0.78) (layer "F.Cu") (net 14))
 (segment (start 162.56 116.586) (end 162.306 116.332) (width 0.78) (layer "F.Cu") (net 14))
 (segment (start 159.512 116.332) (end 155.194 112.014) (width 0.78) (layer "F.Cu") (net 14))
 (segment (start 155.194 112.014) (end 152.439921 112.014) (width 0.78) (layer "F.Cu") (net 14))
 (segment (start 162.56 119.38) (end 162.56 116.586) (width 0.78) (layer "F.Cu") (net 14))
 (segment (start 160.02 118.11) (end 159.258 117.348) (width 0.78) (layer "F.Cu") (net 1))
 (segment (start 145.384389 110.356177) (end 145.384389 109.656178) (width 0.78) (layer "F.Cu") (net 1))
 (segment (start 159.258 117.348) (end 159.14207 117.348) (width 0.78) (layer "F.Cu") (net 1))
 (segment (start 160.02 119.38) (end 160.02 118.11) (width 0.78) (layer "F.Cu") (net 1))
 (segment (start 154.882035 113.087965) (end 148.116177 113.087965) (width 0.78) (layer "F.Cu") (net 1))
 (segment (start 159.14207 117.348) (end 154.882035 113.087965) (width 0.78) (layer "F.Cu") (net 1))
 (segment (start 148.116177 113.087965) (end 145.384389 110.356177) (width 0.78) (layer "F.Cu") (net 1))
 (segment (start 155.96 116.844) (end 155.956 116.84) (width 0.78) (layer "F.Cu") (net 15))
 (segment (start 155.96 115.82) (end 156.09407 115.68593) (width 0.78) (layer "F.Cu") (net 15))
 (segment (start 154.476105 114.067965) (end 144.036221 114.067965) (width 0.78) (layer "F.Cu") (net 15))
 (segment (start 155.956 116.84) (end 155.96 116.836) (width 0.78) (layer "F.Cu") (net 15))
 (segment (start 144.036221 114.067965) (end 140.378956 110.4107) (width 0.78) (layer "F.Cu") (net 15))
 (segment (start 155.96 119.38) (end 155.96 116.844) (width 0.78) (layer "F.Cu") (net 15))
 (segment (start 140.378956 110.4107) (end 140.378956 109.710701) (width 0.78) (layer "F.Cu") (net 15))
 (segment (start 156.09407 115.68593) (end 154.476105 114.067965) (width 0.78) (layer "F.Cu") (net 15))
 (segment (start 155.96 116.836) (end 155.96 115.82) (width 0.78) (layer "F.Cu") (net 15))
 (via (at 155.956 116.84) (size 0.8) (drill 0.4) (layers "F.Cu" "B.Cu") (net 15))
 (segment (start 142.374 117.99) (end 135.30838 110.92438) (width 0.78) (layer "F.Cu") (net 3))
 (segment (start 135.30838 110.92438) (end 135.30838 109.819745) (width 0.78) (layer "F.Cu") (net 3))
 (segment (start 152.03 117.99) (end 142.374 117.99) (width 0.78) (layer "F.Cu") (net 3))
 (segment (start 153.42 119.38) (end 152.03 117.99) (width 0.78) (layer "F.Cu") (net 3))
 (segment (start 137.19305 109.810075) (end 137.18338 109.819745) (width 0.78) (layer "F.Cu") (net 4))
 (segment (start 137.19305 99.877835) (end 137.19305 109.810075) (width 0.78) (layer "F.Cu") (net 4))
 (segment (start 142.27305 99.877835) (end 142.27305 109.691607) (width 0.78) (layer "F.Cu") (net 16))
 (segment (start 142.27305 109.691607) (end 142.253956 109.710701) (width 0.78) (layer "F.Cu") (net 16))
 (segment (start 147.244915 109.641704) (end 147.259389 109.656178) (width 0.78) (layer "F.Cu") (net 2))
 (segment (start 147.244915 99.869085) (end 147.244915 109.641704) (width 0.78) (layer "F.Cu") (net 2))
 (segment (start 152.43305 99.877835) (end 152.43305 109.43213) (width 0.78) (layer "F.Cu") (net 9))
 (segment (start 152.43305 109.43213) (end 152.439009 109.438089) (width 0.78) (layer "F.Cu") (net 9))
 (segment (start 157.51305 99.877835) (end 157.51305 109.485455) (width 0.78) (layer "F.Cu") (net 11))
 (segment (start 157.51305 109.485455) (end 157.520206 109.492611) (width 0.78) (layer "F.Cu") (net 11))
 (segment (start 162.59305 109.320693) (end 162.655924 109.383567) (width 0.78) (layer "F.Cu") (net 10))
 (segment (start 162.59305 99.877835) (end 162.59305 109.320693) (width 0.78) (layer "F.Cu") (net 10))
 (segment (start 167.67305 109.470298) (end 167.650737 109.492611) (width 0.78) (layer "F.Cu") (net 6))
 (segment (start 167.67305 99.877835) (end 167.67305 109.470298) (width 0.78) (layer "F.Cu") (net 6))
 (segment (start 172.783 99.907785) (end 172.75305 99.877835) (width 0.78) (layer "F.Cu") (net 8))
 (segment (start 172.783 109.22) (end 172.783 99.907785) (width 0.78) (layer "F.Cu") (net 8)))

